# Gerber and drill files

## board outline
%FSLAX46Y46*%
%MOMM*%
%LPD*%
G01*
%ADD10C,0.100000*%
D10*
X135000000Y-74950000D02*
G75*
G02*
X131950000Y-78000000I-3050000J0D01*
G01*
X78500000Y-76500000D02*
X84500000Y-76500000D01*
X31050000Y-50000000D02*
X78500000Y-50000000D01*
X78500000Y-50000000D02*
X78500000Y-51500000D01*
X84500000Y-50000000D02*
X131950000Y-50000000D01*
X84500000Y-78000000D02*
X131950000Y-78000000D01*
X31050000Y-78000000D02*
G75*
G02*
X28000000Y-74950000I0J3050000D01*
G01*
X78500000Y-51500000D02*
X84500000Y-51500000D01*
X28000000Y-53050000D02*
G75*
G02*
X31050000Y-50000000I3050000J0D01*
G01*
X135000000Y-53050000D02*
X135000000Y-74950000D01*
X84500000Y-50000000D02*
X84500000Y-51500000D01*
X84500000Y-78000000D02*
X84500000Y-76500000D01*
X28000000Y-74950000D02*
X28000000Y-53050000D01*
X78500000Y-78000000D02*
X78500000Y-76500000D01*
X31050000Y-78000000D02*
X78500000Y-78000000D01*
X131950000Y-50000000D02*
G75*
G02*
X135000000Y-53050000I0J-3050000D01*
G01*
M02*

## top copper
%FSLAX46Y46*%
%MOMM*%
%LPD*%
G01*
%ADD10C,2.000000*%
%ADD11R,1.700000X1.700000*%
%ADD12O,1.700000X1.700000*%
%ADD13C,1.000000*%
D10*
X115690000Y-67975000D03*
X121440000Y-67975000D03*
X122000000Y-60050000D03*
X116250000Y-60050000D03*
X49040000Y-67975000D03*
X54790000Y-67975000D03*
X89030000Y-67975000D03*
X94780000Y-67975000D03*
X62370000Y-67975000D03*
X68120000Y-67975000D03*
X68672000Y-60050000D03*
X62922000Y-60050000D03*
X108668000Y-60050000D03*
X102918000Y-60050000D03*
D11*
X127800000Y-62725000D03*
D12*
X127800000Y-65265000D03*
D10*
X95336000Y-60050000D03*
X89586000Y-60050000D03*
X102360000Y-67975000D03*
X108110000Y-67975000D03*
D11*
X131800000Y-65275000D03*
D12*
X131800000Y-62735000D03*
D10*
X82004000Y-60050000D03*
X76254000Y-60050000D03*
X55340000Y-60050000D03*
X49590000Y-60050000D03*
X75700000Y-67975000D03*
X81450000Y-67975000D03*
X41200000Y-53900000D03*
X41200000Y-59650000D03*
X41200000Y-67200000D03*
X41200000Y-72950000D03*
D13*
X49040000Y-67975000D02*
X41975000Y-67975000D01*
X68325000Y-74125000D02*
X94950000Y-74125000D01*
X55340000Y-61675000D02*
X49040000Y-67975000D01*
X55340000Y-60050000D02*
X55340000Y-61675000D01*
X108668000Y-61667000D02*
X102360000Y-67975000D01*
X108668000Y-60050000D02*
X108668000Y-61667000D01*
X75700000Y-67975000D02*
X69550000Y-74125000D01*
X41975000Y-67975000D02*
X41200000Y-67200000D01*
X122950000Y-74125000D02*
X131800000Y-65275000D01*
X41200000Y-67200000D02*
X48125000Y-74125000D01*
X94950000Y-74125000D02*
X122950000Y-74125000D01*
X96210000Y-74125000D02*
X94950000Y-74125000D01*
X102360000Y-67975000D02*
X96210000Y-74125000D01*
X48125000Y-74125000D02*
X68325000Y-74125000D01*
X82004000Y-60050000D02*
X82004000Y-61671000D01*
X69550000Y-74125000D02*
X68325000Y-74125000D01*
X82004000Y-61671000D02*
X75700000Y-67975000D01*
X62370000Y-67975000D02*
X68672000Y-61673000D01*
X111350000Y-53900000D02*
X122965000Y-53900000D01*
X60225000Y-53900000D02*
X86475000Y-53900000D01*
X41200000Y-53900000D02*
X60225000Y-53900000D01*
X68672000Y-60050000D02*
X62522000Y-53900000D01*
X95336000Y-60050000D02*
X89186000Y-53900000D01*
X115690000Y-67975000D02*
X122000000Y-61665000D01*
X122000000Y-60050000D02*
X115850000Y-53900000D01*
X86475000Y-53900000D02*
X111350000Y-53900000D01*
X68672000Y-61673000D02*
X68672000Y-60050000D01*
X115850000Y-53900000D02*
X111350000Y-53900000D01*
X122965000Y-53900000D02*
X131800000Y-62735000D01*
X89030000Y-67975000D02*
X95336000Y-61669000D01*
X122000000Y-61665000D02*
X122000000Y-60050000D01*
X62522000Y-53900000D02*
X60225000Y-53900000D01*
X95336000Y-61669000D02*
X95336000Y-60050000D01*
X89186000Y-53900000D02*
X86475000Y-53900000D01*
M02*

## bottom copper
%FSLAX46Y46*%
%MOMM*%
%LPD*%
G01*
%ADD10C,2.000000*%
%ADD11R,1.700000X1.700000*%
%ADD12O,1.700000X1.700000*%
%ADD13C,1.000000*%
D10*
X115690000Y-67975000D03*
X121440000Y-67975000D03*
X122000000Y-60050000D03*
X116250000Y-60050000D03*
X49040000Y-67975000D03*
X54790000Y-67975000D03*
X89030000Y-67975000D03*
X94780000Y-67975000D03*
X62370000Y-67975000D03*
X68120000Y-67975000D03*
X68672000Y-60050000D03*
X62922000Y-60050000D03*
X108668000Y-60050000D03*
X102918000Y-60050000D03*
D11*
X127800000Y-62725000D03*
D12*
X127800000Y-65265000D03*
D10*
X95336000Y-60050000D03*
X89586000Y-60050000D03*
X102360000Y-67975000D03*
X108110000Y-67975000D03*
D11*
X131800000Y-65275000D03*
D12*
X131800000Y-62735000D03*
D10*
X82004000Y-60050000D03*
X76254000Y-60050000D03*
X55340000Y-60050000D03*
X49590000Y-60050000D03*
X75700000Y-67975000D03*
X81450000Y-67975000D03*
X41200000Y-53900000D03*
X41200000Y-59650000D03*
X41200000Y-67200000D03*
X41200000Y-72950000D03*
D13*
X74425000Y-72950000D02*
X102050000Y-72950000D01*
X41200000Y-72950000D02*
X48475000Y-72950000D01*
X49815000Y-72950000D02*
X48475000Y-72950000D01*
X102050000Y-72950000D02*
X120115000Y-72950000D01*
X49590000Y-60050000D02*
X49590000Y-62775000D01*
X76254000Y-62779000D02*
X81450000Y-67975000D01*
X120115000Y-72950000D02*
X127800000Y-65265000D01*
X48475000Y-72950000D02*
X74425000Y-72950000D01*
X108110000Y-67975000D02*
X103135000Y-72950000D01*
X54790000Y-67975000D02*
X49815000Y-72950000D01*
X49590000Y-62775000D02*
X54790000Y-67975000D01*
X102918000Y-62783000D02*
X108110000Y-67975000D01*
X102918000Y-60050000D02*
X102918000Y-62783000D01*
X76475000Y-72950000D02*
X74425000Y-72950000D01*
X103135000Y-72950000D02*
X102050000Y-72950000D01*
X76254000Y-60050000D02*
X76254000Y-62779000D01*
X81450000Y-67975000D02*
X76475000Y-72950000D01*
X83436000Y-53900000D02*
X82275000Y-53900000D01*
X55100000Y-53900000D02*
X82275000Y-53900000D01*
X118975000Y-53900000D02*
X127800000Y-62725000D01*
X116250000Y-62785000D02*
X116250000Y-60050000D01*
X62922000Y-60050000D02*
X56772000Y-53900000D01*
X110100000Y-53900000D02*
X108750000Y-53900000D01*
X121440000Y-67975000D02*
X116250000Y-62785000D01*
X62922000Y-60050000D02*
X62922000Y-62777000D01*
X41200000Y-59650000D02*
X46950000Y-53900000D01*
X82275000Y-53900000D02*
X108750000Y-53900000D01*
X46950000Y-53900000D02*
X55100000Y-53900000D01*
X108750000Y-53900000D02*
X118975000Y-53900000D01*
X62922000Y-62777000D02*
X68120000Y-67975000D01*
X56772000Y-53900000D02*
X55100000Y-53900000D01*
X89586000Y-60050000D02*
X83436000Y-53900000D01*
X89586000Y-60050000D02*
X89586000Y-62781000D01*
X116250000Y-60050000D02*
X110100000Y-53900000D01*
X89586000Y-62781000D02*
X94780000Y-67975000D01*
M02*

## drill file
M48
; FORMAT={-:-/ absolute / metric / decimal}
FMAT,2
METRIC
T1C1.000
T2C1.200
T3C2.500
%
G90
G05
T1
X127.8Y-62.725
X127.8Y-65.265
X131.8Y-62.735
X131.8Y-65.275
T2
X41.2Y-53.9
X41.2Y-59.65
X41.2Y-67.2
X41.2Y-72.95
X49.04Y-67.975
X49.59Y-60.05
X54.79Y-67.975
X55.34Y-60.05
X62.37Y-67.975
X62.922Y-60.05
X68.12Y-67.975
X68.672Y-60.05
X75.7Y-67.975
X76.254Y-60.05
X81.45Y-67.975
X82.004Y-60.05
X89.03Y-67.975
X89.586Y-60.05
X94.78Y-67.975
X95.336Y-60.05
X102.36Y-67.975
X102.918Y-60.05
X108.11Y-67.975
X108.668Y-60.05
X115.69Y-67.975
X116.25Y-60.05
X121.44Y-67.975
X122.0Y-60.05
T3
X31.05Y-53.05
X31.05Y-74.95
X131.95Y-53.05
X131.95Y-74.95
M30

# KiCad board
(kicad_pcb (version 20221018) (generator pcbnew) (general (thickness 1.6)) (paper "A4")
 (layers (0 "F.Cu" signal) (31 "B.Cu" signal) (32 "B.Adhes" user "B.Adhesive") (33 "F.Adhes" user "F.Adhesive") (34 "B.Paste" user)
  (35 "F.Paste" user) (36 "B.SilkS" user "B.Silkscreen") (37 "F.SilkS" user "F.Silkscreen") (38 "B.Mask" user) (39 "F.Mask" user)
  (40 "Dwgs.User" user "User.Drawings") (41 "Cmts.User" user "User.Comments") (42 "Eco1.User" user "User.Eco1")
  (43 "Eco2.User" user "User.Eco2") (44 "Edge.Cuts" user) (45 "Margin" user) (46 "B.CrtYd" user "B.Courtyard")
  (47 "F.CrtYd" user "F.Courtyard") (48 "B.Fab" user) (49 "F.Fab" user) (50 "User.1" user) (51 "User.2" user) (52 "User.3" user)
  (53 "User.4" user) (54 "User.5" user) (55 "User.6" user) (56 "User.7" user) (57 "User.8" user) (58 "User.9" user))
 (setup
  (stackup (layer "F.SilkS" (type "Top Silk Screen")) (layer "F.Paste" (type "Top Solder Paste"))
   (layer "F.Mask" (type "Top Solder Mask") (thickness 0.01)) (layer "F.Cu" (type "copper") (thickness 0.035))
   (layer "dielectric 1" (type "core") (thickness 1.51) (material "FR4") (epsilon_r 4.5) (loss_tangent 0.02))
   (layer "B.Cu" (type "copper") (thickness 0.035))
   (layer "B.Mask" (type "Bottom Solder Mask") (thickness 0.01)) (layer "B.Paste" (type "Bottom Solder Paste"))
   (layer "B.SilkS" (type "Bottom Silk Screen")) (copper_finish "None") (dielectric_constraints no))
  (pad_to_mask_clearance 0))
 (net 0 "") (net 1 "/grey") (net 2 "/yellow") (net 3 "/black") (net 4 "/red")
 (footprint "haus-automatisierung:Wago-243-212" (layer "F.Cu") (at 113.04 64.575)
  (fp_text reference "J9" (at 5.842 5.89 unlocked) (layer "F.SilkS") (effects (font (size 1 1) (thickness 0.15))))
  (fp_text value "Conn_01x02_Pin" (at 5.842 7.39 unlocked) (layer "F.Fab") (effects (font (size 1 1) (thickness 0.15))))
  (pad "1" thru_hole circle (at 2.65 3.4) (size 2 2) (drill 1.2) (layers "*.Cu" "*.Mask") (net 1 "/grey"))
  (pad "2" thru_hole circle (at 8.4 3.4) (size 2 2) (drill 1.2) (layers "*.Cu" "*.Mask") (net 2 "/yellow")))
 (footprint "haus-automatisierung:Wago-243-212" (layer "F.Cu") (at 124.65 63.45 180)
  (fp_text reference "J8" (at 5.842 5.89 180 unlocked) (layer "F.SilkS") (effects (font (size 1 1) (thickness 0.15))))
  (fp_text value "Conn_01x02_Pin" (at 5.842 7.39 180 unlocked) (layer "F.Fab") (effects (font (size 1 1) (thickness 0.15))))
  (pad "1" thru_hole circle (at 2.65 3.4 180) (size 2 2) (drill 1.2) (layers "*.Cu" "*.Mask") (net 1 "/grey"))
  (pad "2" thru_hole circle (at 8.4 3.4 180) (size 2 2) (drill 1.2) (layers "*.Cu" "*.Mask") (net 2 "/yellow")))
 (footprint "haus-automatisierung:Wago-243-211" (layer "F.Cu") (at 46.39 64.575)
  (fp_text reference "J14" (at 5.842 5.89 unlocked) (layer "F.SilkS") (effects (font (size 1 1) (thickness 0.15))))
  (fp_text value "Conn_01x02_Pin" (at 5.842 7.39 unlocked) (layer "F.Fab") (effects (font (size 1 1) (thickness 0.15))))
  (pad "1" thru_hole circle (at 2.65 3.4) (size 2 2) (drill 1.2) (layers "*.Cu" "*.Mask") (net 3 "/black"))
  (pad "2" thru_hole circle (at 8.4 3.4) (size 2 2) (drill 1.2) (layers "*.Cu" "*.Mask") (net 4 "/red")))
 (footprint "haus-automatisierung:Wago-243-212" (layer "F.Cu") (at 86.38 64.575)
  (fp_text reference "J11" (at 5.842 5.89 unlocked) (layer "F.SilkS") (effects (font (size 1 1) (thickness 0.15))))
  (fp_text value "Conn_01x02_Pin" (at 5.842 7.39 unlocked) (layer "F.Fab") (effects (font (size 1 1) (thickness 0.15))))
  (pad "1" thru_hole circle (at 2.65 3.4) (size 2 2) (drill 1.2) (layers "*.Cu" "*.Mask") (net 1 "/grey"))
  (pad "2" thru_hole circle (at 8.4 3.4) (size 2 2) (drill 1.2) (layers "*.Cu" "*.Mask") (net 2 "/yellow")))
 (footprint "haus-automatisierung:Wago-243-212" (layer "F.Cu") (at 59.72 64.575)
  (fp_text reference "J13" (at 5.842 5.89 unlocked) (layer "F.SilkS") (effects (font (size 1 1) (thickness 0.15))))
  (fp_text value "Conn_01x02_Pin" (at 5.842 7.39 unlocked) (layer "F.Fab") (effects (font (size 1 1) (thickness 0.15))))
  (pad "1" thru_hole circle (at 2.65 3.4) (size 2 2) (drill 1.2) (layers "*.Cu" "*.Mask") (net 1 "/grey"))
  (pad "2" thru_hole circle (at 8.4 3.4) (size 2 2) (drill 1.2) (layers "*.Cu" "*.Mask") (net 2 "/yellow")))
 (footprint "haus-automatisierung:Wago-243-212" (layer "F.Cu") (at 71.322 63.45 180)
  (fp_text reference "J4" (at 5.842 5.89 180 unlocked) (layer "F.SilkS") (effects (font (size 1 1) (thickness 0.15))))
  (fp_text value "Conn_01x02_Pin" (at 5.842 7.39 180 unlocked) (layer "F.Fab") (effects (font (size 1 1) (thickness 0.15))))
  (pad "1" thru_hole circle (at 2.65 3.4 180) (size 2 2) (drill 1.2) (layers "*.Cu" "*.Mask") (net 1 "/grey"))
  (pad "2" thru_hole circle (at 8.4 3.4 180) (size 2 2) (drill 1.2) (layers "*.Cu" "*.Mask") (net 2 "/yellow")))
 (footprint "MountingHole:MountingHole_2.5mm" (layer "F.Cu") (at 131.95 53.05)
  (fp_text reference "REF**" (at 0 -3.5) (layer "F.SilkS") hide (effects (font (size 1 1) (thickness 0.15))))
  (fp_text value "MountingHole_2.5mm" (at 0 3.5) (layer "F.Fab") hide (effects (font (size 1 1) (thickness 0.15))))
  (pad "" np_thru_hole circle (at 0 0) (size 2.5 2.5) (drill 2.5) (layers "*.Cu" "*.Mask")))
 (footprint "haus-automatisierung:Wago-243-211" (layer "F.Cu") (at 111.318 63.45 180)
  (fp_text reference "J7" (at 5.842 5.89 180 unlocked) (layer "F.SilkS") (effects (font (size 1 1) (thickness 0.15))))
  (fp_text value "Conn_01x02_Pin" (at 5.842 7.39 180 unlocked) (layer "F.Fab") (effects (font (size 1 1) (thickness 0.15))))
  (pad "1" thru_hole circle (at 2.65 3.4 180) (size 2 2) (drill 1.2) (layers "*.Cu" "*.Mask") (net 3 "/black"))
  (pad "2" thru_hole circle (at 8.4 3.4 180) (size 2 2) (drill 1.2) (layers "*.Cu" "*.Mask") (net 4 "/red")))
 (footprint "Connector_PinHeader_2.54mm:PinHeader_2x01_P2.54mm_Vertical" (layer "F.Cu") (at 127.8 62.725 -90)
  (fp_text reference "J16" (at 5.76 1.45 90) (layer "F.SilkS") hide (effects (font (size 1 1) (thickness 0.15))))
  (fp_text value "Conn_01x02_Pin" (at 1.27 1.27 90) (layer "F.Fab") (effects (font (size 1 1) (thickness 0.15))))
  (pad "1" thru_hole rect (at 0 0 270) (size 1.7 1.7) (drill 1) (layers "*.Cu" "*.Mask") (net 2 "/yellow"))
  (pad "2" thru_hole oval (at 2.54 0 270) (size 1.7 1.7) (drill 1) (layers "*.Cu" "*.Mask") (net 4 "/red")))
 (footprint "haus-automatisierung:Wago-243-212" (layer "F.Cu") (at 97.986 63.45 180)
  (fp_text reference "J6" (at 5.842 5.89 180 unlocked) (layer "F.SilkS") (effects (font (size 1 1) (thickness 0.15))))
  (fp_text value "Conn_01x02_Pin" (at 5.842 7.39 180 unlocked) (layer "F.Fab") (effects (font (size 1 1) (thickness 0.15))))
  (pad "1" thru_hole circle (at 2.65 3.4 180) (size 2 2) (drill 1.2) (layers "*.Cu" "*.Mask") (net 1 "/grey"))
  (pad "2" thru_hole circle (at 8.4 3.4 180) (size 2 2) (drill 1.2) (layers "*.Cu" "*.Mask") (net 2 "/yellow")))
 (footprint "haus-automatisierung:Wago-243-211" (layer "F.Cu") (at 99.71 64.575)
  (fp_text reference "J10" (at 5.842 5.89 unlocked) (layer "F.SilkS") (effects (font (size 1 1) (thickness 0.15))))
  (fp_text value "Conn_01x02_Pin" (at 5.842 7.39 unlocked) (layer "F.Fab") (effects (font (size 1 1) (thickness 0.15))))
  (pad "1" thru_hole circle (at 2.65 3.4) (size 2 2) (drill 1.2) (layers "*.Cu" "*.Mask") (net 3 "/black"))
  (pad "2" thru_hole circle (at 8.4 3.4) (size 2 2) (drill 1.2) (layers "*.Cu" "*.Mask") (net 4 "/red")))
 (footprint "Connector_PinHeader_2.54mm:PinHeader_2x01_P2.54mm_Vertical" (layer "F.Cu") (at 131.8 65.275 90)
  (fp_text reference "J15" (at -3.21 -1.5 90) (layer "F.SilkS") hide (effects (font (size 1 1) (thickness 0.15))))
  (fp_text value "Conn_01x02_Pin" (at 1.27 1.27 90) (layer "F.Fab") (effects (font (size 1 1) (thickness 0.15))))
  (pad "1" thru_hole rect (at 0 0 90) (size 1.7 1.7) (drill 1) (layers "*.Cu" "*.Mask") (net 3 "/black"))
  (pad "2" thru_hole oval (at 2.54 0 90) (size 1.7 1.7) (drill 1) (layers "*.Cu" "*.Mask") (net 1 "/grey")))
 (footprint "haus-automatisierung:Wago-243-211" (layer "F.Cu") (at 84.654 63.45 180)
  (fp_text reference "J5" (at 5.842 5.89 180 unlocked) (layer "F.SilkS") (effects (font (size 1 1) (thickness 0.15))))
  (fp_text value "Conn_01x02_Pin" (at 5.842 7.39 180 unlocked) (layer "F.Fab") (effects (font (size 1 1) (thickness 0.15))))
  (pad "1" thru_hole circle (at 2.65 3.4 180) (size 2 2) (drill 1.2) (layers "*.Cu" "*.Mask") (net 3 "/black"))
  (pad "2" thru_hole circle (at 8.4 3.4 180) (size 2 2) (drill 1.2) (layers "*.Cu" "*.Mask") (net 4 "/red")))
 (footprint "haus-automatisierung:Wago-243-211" (layer "F.Cu") (at 57.99 63.45 180)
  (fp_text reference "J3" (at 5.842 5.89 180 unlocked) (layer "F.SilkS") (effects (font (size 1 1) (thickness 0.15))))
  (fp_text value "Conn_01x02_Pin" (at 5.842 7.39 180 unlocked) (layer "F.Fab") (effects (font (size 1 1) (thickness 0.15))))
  (pad "1" thru_hole circle (at 2.65 3.4 180) (size 2 2) (drill 1.2) (layers "*.Cu" "*.Mask") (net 3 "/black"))
  (pad "2" thru_hole circle (at 8.4 3.4 180) (size 2 2) (drill 1.2) (layers "*.Cu" "*.Mask") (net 4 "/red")))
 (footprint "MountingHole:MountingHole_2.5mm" (layer "F.Cu") (at 31.05 53.05)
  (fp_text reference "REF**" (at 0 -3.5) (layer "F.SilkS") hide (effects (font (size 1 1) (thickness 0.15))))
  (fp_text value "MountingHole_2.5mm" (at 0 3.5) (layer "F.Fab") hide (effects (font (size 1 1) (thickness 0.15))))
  (pad "" np_thru_hole circle (at 0 0) (size 2.5 2.5) (drill 2.5) (layers "*.Cu" "*.Mask")))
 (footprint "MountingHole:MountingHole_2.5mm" (layer "F.Cu") (at 131.95 74.95)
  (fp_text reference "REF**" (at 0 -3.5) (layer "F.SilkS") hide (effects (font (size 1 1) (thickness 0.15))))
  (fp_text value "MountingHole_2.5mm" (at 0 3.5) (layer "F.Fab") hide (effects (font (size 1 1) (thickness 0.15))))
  (pad "" np_thru_hole circle (at 0 0) (size 2.5 2.5) (drill 2.5) (layers "*.Cu" "*.Mask")))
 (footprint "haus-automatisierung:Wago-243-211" (layer "F.Cu") (at 73.05 64.575)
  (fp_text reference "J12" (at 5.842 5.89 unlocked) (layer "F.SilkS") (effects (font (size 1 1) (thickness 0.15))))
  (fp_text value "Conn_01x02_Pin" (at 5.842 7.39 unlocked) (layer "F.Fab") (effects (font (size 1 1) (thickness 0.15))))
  (pad "1" thru_hole circle (at 2.65 3.4) (size 2 2) (drill 1.2) (layers "*.Cu" "*.Mask") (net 3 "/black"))
  (pad "2" thru_hole circle (at 8.4 3.4) (size 2 2) (drill 1.2) (layers "*.Cu" "*.Mask") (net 4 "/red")))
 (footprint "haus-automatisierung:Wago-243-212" (layer "F.Cu") (at 44.6 51.25 -90)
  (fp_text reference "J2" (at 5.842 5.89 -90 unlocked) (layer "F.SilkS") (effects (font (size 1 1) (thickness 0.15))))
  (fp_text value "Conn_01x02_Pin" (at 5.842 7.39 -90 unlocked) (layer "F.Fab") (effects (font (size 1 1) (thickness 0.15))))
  (pad "1" thru_hole circle (at 2.65 3.4 270) (size 2 2) (drill 1.2) (layers "*.Cu" "*.Mask") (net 1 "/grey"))
  (pad "2" thru_hole circle (at 8.4 3.4 270) (size 2 2) (drill 1.2) (layers "*.Cu" "*.Mask") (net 2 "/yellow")))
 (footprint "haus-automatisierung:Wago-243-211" (layer "F.Cu") (at 44.6 64.55 -90)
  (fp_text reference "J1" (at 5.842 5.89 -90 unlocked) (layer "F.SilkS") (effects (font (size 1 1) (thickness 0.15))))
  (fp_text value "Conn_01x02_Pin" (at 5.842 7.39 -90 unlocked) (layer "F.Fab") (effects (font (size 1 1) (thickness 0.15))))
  (pad "1" thru_hole circle (at 2.65 3.4 270) (size 2 2) (drill 1.2) (layers "*.Cu" "*.Mask") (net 3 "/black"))
  (pad "2" thru_hole circle (at 8.4 3.4 270) (size 2 2) (drill 1.2) (layers "*.Cu" "*.Mask") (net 4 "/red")))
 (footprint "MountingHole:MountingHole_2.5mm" (layer "F.Cu") (at 31.05 74.95)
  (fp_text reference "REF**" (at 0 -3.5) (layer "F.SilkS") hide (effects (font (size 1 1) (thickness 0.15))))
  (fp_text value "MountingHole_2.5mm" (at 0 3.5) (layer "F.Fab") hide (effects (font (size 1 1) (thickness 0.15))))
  (pad "" np_thru_hole circle (at 0 0) (size 2.5 2.5) (drill 2.5) (layers "*.Cu" "*.Mask")))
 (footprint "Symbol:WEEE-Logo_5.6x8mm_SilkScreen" (layer "B.Cu") (at 121.5 64 -90)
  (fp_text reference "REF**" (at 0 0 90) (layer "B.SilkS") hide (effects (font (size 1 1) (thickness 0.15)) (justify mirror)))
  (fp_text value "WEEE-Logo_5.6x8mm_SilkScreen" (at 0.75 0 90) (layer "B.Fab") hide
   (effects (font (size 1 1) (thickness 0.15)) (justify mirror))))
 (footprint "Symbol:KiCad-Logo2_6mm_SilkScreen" (layer "B.Cu") (at 34.4 64 -90)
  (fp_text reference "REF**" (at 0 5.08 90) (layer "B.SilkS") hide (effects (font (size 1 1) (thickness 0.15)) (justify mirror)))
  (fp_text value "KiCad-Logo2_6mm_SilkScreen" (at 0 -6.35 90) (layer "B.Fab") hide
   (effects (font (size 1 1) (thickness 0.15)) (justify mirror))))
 (gr_arc (start 135 74.95) (mid 134.106676 77.106676) (end 131.95 78) (stroke (width 0.1) (type default)) (layer "Edge.Cuts"))
 (gr_line (start 78.5 76.5) (end 84.5 76.5) (stroke (width 0.1) (type default)) (layer "Edge.Cuts"))
 (gr_line (start 31.05 50) (end 78.5 50) (stroke (width 0.1) (type default)) (layer "Edge.Cuts"))
 (gr_line (start 78.5 50) (end 78.5 51.5) (stroke (width 0.1) (type default)) (layer "Edge.Cuts"))
 (gr_line (start 84.5 50) (end 131.95 50) (stroke (width 0.1) (type default)) (layer "Edge.Cuts"))
 (gr_line (start 84.5 78) (end 131.95 78) (stroke (width 0.1) (type default)) (layer "Edge.Cuts"))
 (gr_arc (start 31.05 78) (mid 28.893324 77.106676) (end 28 74.95) (stroke (width 0.1) (type default)) (layer "Edge.Cuts"))
 (gr_line (start 78.5 51.5) (end 84.5 51.5) (stroke (width 0.1) (type default)) (layer "Edge.Cuts"))
 (gr_arc (start 28 53.05) (mid 28.893324 50.893324) (end 31.05 50) (stroke (width 0.1) (type default)) (layer "Edge.Cuts"))
 (gr_line (start 135 53.05) (end 135 74.95) (stroke (width 0.1) (type default)) (layer "Edge.Cuts"))
 (gr_line (start 84.5 50) (end 84.5 51.5) (stroke (width 0.1) (type default)) (layer "Edge.Cuts"))
 (gr_line (start 84.5 78) (end 84.5 76.5) (stroke (width 0.1) (type default)) (layer "Edge.Cuts"))
 (gr_line (start 28 74.95) (end 28 53.05) (stroke (width 0.1) (type default)) (layer "Edge.Cuts"))
 (gr_line (start 78.5 78) (end 78.5 76.5) (stroke (width 0.1) (type default)) (layer "Edge.Cuts"))
 (gr_line (start 31.05 78) (end 78.5 78) (stroke (width 0.1) (type default)) (layer "Edge.Cuts"))
 (gr_arc (start 131.95 50) (mid 134.106676 50.893324) (end 135 53.05) (stroke (width 0.1) (type default)) (layer "Edge.Cuts"))
 (segment (start 49.04 67.975) (end 41.975 67.975) (width 1) (layer "F.Cu") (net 3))
 (segment (start 68.325 74.125) (end 94.95 74.125) (width 1) (layer "F.Cu") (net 3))
 (segment (start 55.34 61.675) (end 49.04 67.975) (width 1) (layer "F.Cu") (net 3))
 (segment (start 55.34 60.05) (end 55.34 61.675) (width 1) (layer "F.Cu") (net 3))
 (segment (start 108.668 61.667) (end 102.36 67.975) (width 1) (layer "F.Cu") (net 3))
 (segment (start 108.668 60.05) (end 108.668 61.667) (width 1) (layer "F.Cu") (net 3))
 (segment (start 75.7 67.975) (end 69.55 74.125) (width 1) (layer "F.Cu") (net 3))
 (segment (start 41.975 67.975) (end 41.2 67.2) (width 1) (layer "F.Cu") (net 3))
 (segment (start 122.95 74.125) (end 131.8 65.275) (width 1) (layer "F.Cu") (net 3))
 (segment (start 41.2 67.2) (end 48.125 74.125) (width 1) (layer "F.Cu") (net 3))
 (segment (start 94.95 74.125) (end 122.95 74.125) (width 1) (layer "F.Cu") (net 3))
 (segment (start 96.21 74.125) (end 94.95 74.125) (width 1) (layer "F.Cu") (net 3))
 (segment (start 102.36 67.975) (end 96.21 74.125) (width 1) (layer "F.Cu") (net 3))
 (segment (start 48.125 74.125) (end 68.325 74.125) (width 1) (layer "F.Cu") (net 3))
 (segment (start 82.004 60.05) (end 82.004 61.671) (width 1) (layer "F.Cu") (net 3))
 (segment (start 69.55 74.125) (end 68.325 74.125) (width 1) (layer "F.Cu") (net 3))
 (segment (start 82.004 61.671) (end 75.7 67.975) (width 1) (layer "F.Cu") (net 3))
 (segment (start 74.425 72.95) (end 102.05 72.95) (width 1) (layer "B.Cu") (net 4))
 (segment (start 41.2 72.95) (end 48.475 72.95) (width 1) (layer "B.Cu") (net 4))
 (segment (start 49.815 72.95) (end 48.475 72.95) (width 1) (layer "B.Cu") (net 4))
 (segment (start 102.05 72.95) (end 120.115 72.95) (width 1) (layer "B.Cu") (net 4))
 (segment (start 49.59 60.05) (end 49.59 62.775) (width 1) (layer "B.Cu") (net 4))
 (segment (start 76.254 62.779) (end 81.45 67.975) (width 1) (layer "B.Cu") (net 4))
 (segment (start 120.115 72.95) (end 127.8 65.265) (width 1) (layer "B.Cu") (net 4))
 (segment (start 48.475 72.95) (end 74.425 72.95) (width 1) (layer "B.Cu") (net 4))
 (segment (start 108.11 67.975) (end 103.135 72.95) (width 1) (layer "B.Cu") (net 4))
 (segment (start 54.79 67.975) (end 49.815 72.95) (width 1) (layer "B.Cu") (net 4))
 (segment (start 49.59 62.775) (end 54.79 67.975) (width 1) (layer "B.Cu") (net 4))
 (segment (start 102.918 62.783) (end 108.11 67.975) (width 1) (layer "B.Cu") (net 4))
 (segment (start 102.918 60.05) (end 102.918 62.783) (width 1) (layer "B.Cu") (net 4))
 (segment (start 76.475 72.95) (end 74.425 72.95) (width 1) (layer "B.Cu") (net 4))
 (segment (start 103.135 72.95) (end 102.05 72.95) (width 1) (layer "B.Cu") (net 4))
 (segment (start 76.254 60.05) (end 76.254 62.779) (width 1) (layer "B.Cu") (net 4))
 (segment (start 81.45 67.975) (end 76.475 72.95) (width 1) (layer "B.Cu") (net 4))
 (segment (start 62.37 67.975) (end 68.672 61.673) (width 1) (layer "F.Cu") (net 1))
 (segment (start 111.35 53.9) (end 122.965 53.9) (width 1) (layer "F.Cu") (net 1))
 (segment (start 60.225 53.9) (end 86.475 53.9) (width 1) (layer "F.Cu") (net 1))
 (segment (start 41.2 53.9) (end 60.225 53.9) (width 1) (layer "F.Cu") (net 1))
 (segment (start 68.672 60.05) (end 62.522 53.9) (width 1) (layer "F.Cu") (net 1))
 (segment (start 95.336 60.05) (end 89.186 53.9) (width 1) (layer "F.Cu") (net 1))
 (segment (start 115.69 67.975) (end 122 61.665) (width 1) (layer "F.Cu") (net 1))
 (segment (start 122 60.05) (end 115.85 53.9) (width 1) (layer "F.Cu") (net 1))
 (segment (start 86.475 53.9) (end 111.35 53.9) (width 1) (layer "F.Cu") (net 1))
 (segment (start 68.672 61.673) (end 68.672 60.05) (width 1) (layer "F.Cu") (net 1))
 (segment (start 115.85 53.9) (end 111.35 53.9) (width 1) (layer "F.Cu") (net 1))
 (segment (start 122.965 53.9) (end 131.8 62.735) (width 1) (layer "F.Cu") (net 1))
 (segment (start 89.03 67.975) (end 95.336 61.669) (width 1) (layer "F.Cu") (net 1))
 (segment (start 122 61.665) (end 122 60.05) (width 1) (layer "F.Cu") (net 1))
 (segment (start 62.522 53.9) (end 60.225 53.9) (width 1) (layer "F.Cu") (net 1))
 (segment (start 95.336 61.669) (end 95.336 60.05) (width 1) (layer "F.Cu") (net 1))
 (segment (start 89.186 53.9) (end 86.475 53.9) (width 1) (layer "F.Cu") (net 1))
 (segment (start 83.436 53.9) (end 82.275 53.9) (width 1) (layer "B.Cu") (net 2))
 (segment (start 55.1 53.9) (end 82.275 53.9) (width 1) (layer "B.Cu") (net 2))
 (segment (start 118.975 53.9) (end 127.8 62.725) (width 1) (layer "B.Cu") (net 2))
 (segment (start 116.25 62.785) (end 116.25 60.05) (width 1) (layer "B.Cu") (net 2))
 (segment (start 62.922 60.05) (end 56.772 53.9) (width 1) (layer "B.Cu") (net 2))
 (segment (start 110.1 53.9) (end 108.75 53.9) (width 1) (layer "B.Cu") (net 2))
 (segment (start 121.44 67.975) (end 116.25 62.785) (width 1) (layer "B.Cu") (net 2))
 (segment (start 62.922 60.05) (end 62.922 62.777) (width 1) (layer "B.Cu") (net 2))
 (segment (start 41.2 59.65) (end 46.95 53.9) (width 1) (layer "B.Cu") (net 2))
 (segment (start 82.275 53.9) (end 108.75 53.9) (width 1) (layer "B.Cu") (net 2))
 (segment (start 46.95 53.9) (end 55.1 53.9) (width 1) (layer "B.Cu") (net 2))
 (segment (start 108.75 53.9) (end 118.975 53.9) (width 1) (layer "B.Cu") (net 2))
 (segment (start 62.922 62.777) (end 68.12 67.975) (width 1) (layer "B.Cu") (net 2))
 (segment (start 56.772 53.9) (end 55.1 53.9) (width 1) (layer "B.Cu") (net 2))
 (segment (start 89.586 60.05) (end 83.436 53.9) (width 1) (layer "B.Cu") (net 2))
 (segment (start 89.586 60.05) (end 89.586 62.781) (width 1) (layer "B.Cu") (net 2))
 (segment (start 116.25 60.05) (end 110.1 53.9) (width 1) (layer "B.Cu") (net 2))
 (segment (start 89.586 62.781) (end 94.78 67.975) (width 1) (layer "B.Cu") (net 2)))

